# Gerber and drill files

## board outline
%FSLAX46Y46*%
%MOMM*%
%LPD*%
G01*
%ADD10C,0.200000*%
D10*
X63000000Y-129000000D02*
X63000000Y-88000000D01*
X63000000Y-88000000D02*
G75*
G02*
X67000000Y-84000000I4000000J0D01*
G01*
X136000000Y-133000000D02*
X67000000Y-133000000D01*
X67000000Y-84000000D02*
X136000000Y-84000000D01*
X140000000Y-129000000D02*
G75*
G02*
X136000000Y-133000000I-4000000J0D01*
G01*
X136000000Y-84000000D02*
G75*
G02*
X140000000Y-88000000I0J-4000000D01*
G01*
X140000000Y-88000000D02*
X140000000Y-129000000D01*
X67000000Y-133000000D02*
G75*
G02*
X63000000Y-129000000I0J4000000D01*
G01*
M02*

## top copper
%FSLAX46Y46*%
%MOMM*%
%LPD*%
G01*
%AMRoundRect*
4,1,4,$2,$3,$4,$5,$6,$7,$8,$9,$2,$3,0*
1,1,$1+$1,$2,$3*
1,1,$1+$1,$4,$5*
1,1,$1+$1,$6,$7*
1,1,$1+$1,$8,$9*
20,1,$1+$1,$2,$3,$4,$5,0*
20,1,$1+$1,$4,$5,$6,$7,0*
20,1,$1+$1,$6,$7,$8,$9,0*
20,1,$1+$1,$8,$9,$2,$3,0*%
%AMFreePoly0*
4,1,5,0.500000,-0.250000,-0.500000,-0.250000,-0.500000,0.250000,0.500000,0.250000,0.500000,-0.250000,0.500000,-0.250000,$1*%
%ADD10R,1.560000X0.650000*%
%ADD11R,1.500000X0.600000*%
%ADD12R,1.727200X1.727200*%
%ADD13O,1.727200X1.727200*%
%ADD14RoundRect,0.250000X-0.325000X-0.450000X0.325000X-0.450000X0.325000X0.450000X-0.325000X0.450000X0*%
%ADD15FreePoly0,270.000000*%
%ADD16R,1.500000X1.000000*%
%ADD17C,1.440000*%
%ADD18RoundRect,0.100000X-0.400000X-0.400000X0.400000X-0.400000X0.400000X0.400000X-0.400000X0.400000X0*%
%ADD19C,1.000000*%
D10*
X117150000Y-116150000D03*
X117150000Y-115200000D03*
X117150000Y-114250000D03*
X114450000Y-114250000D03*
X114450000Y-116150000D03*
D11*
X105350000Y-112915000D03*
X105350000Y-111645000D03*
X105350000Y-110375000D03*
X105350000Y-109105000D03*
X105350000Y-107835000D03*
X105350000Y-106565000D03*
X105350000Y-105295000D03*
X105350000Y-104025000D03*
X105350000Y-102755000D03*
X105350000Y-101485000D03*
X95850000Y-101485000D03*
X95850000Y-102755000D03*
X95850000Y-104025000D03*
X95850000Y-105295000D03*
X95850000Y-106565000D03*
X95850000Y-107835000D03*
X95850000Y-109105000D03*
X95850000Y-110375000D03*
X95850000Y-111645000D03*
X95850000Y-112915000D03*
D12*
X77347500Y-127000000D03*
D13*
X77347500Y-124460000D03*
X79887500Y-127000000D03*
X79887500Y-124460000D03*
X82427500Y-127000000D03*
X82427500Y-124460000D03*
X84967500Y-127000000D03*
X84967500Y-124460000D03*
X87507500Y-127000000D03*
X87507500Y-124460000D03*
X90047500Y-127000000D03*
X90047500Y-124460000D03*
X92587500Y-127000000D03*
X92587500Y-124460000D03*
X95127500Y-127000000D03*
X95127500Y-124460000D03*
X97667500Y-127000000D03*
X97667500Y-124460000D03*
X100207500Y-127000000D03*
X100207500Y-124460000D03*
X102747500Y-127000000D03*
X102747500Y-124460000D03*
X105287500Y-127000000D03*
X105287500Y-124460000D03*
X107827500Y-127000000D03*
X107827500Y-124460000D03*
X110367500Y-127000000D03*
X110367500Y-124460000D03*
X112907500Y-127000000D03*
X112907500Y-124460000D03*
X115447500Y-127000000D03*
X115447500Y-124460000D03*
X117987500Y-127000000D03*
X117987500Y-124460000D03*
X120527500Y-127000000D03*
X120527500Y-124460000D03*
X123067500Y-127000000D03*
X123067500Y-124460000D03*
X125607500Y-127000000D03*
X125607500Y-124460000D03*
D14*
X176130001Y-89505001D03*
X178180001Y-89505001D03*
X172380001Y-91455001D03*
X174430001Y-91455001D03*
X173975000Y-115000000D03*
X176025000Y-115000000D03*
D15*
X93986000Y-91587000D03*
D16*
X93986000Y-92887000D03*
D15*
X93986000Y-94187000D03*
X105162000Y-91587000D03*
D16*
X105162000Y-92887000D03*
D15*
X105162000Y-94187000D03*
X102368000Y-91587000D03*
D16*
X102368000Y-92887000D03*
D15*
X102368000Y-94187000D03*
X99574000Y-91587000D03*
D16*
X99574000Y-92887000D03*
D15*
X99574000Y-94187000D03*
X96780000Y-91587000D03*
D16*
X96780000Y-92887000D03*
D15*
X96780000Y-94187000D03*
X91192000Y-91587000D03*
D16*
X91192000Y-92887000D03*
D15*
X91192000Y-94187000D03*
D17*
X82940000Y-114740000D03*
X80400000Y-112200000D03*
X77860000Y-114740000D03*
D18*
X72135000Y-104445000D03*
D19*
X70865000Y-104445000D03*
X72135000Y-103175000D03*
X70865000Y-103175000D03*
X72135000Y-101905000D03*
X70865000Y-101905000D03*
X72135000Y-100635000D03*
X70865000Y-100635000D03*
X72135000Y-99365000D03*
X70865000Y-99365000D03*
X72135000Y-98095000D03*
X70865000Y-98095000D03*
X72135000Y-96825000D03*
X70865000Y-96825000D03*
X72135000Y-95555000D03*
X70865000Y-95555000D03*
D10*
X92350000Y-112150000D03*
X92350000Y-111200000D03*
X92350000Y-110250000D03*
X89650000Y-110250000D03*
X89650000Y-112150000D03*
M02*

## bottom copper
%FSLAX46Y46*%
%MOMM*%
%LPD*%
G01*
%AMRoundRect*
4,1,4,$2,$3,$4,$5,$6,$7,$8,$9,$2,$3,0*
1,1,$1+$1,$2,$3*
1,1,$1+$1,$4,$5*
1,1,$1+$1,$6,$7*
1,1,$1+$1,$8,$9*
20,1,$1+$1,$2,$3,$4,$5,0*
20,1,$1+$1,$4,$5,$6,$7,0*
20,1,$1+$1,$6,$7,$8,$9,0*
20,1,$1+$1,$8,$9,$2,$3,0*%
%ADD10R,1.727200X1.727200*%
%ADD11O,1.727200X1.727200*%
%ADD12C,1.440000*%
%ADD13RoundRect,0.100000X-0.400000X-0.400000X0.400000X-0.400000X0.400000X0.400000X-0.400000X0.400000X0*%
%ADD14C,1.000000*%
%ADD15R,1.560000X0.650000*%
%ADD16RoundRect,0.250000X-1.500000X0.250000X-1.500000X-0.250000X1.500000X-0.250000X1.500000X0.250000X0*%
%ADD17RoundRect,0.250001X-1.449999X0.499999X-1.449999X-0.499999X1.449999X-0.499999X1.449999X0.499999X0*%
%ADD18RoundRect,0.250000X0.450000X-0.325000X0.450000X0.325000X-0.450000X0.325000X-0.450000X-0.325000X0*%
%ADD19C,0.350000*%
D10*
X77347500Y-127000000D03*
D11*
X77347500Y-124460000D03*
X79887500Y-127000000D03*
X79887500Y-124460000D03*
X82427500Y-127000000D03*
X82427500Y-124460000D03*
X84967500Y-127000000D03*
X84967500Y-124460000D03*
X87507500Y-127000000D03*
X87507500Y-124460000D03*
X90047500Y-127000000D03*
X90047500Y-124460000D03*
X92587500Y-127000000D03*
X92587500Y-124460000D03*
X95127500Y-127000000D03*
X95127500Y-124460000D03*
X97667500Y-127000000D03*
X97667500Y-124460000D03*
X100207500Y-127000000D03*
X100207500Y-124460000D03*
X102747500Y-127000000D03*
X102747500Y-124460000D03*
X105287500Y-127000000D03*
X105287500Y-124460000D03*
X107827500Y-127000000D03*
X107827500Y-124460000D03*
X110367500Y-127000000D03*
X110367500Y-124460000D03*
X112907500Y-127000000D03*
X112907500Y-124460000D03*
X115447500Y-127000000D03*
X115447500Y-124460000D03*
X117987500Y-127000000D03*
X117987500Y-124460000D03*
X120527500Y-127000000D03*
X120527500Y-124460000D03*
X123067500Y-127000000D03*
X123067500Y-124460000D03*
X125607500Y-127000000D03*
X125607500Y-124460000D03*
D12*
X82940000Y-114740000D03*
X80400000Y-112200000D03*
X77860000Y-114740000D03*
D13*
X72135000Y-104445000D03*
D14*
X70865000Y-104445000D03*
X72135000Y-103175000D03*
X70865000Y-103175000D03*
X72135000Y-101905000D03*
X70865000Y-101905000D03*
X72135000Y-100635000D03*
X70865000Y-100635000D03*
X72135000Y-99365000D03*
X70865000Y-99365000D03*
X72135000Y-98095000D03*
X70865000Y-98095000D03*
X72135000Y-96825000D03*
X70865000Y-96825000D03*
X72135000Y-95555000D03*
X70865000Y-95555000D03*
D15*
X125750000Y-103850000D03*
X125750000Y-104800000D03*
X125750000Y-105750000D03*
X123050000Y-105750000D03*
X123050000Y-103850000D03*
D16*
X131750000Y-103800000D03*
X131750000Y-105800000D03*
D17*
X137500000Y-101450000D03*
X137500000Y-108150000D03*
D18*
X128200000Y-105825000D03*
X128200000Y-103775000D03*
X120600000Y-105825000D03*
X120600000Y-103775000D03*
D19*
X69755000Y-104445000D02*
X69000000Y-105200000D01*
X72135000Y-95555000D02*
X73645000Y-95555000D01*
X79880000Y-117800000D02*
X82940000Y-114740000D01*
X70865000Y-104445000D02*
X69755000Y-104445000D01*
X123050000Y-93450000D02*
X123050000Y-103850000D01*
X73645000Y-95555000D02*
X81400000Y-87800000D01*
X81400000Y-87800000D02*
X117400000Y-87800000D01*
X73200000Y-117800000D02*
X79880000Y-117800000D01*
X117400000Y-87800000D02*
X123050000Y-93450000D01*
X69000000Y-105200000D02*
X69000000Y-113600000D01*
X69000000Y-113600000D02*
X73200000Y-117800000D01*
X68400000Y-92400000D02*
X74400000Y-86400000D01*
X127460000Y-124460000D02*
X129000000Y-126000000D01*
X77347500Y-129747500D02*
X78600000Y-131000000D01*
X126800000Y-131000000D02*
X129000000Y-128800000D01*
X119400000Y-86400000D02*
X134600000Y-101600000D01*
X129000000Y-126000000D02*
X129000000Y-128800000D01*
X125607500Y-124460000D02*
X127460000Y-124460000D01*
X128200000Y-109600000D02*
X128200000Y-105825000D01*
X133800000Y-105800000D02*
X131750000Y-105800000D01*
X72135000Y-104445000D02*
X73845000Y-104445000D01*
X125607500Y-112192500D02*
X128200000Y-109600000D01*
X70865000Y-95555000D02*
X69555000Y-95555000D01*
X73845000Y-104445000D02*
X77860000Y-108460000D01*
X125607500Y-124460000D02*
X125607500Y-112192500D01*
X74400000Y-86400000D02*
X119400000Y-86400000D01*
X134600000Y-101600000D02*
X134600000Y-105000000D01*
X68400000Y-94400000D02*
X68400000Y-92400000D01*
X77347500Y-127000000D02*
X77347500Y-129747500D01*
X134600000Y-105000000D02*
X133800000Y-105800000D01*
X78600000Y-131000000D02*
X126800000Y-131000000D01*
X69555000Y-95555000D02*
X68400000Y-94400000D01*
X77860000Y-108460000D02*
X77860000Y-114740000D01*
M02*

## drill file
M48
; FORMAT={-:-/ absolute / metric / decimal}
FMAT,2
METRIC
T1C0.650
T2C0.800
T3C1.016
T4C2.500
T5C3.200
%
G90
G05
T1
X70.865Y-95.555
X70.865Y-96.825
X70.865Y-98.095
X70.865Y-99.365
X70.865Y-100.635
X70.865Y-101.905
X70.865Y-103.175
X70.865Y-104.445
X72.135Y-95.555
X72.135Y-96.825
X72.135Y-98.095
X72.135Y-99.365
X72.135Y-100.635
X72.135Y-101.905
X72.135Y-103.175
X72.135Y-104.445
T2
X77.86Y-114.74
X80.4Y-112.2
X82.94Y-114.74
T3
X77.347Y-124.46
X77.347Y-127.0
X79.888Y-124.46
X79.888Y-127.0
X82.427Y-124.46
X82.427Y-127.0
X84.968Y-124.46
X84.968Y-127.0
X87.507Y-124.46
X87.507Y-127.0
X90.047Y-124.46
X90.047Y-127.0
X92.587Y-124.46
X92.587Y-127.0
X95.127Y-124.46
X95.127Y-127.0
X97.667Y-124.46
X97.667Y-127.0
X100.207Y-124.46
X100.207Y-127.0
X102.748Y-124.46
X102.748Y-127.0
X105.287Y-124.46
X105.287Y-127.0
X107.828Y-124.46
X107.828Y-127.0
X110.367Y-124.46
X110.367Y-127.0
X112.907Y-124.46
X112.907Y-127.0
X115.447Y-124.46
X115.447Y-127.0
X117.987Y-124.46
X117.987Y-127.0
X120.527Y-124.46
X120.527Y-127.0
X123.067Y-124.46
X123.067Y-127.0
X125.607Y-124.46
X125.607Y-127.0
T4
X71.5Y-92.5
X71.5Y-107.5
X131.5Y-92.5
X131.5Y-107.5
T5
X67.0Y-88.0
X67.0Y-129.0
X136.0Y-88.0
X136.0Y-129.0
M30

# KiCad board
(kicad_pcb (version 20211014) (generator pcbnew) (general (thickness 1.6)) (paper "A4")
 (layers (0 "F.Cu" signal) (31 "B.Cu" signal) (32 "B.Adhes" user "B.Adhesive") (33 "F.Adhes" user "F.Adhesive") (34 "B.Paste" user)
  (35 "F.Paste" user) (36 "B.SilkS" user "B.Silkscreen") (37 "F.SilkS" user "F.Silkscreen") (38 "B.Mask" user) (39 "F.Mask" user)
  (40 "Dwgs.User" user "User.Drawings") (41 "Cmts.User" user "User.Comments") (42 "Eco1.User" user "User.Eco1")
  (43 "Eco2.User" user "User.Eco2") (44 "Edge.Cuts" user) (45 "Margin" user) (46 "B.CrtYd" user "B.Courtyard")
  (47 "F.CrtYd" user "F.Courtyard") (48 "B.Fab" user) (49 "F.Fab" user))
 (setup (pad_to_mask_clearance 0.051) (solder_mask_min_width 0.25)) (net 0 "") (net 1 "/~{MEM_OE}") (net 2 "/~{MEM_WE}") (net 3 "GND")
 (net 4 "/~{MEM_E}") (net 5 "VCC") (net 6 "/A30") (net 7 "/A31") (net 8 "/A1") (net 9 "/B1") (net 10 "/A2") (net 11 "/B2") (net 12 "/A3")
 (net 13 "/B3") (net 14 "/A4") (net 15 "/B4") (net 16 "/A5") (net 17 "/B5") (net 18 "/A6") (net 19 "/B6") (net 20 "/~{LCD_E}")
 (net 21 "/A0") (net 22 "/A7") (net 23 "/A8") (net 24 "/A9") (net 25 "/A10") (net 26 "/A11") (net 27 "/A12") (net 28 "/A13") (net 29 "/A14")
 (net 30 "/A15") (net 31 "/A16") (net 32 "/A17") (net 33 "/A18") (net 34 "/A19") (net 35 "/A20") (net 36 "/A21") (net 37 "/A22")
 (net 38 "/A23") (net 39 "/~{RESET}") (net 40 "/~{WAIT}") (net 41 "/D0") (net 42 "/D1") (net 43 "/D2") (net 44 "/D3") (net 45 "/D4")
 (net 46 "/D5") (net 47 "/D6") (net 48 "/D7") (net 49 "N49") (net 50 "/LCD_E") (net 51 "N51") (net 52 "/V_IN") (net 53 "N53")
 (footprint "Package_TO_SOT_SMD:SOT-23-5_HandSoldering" (layer "F.Cu") (at 115.8 115.2 180)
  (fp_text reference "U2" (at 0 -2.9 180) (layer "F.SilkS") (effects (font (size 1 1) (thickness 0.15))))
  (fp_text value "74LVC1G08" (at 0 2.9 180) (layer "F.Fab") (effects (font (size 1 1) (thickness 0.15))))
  (pad "1" smd rect locked (at -1.35 -0.95 180) (size 1.56 0.65) (layers "F.Cu" "F.Paste" "F.Mask") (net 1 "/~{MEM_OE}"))
  (pad "2" smd rect locked (at -1.35 0 180) (size 1.56 0.65) (layers "F.Cu" "F.Paste" "F.Mask") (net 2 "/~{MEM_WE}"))
  (pad "3" smd rect locked (at -1.35 0.95 180) (size 1.56 0.65) (layers "F.Cu" "F.Paste" "F.Mask") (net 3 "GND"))
  (pad "4" smd rect locked (at 1.35 0.95 180) (size 1.56 0.65) (layers "F.Cu" "F.Paste" "F.Mask") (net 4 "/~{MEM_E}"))
  (pad "5" smd rect locked (at 1.35 -0.95 180) (size 1.56 0.65) (layers "F.Cu" "F.Paste" "F.Mask") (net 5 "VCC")))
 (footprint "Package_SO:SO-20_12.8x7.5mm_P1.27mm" (layer "F.Cu") (at 100.6 107.2 180)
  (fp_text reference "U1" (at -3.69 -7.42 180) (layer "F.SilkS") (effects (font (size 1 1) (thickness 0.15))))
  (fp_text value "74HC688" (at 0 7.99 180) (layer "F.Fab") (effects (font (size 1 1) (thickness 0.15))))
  (pad "1" smd rect locked (at -4.75 -5.715 180) (size 1.5 0.6) (layers "F.Cu" "F.Paste" "F.Mask") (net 4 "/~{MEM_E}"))
  (pad "2" smd rect locked (at -4.75 -4.445 180) (size 1.5 0.6) (layers "F.Cu" "F.Paste" "F.Mask") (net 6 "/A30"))
  (pad "3" smd rect locked (at -4.75 -3.175 180) (size 1.5 0.6) (layers "F.Cu" "F.Paste" "F.Mask") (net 5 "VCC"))
  (pad "4" smd rect locked (at -4.75 -1.905 180) (size 1.5 0.6) (layers "F.Cu" "F.Paste" "F.Mask") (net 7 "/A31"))
  (pad "5" smd rect locked (at -4.75 -0.635 180) (size 1.5 0.6) (layers "F.Cu" "F.Paste" "F.Mask") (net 3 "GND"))
  (pad "6" smd rect locked (at -4.75 0.635 180) (size 1.5 0.6) (layers "F.Cu" "F.Paste" "F.Mask") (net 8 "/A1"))
  (pad "7" smd rect locked (at -4.75 1.905 180) (size 1.5 0.6) (layers "F.Cu" "F.Paste" "F.Mask") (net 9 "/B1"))
  (pad "8" smd rect locked (at -4.75 3.175 180) (size 1.5 0.6) (layers "F.Cu" "F.Paste" "F.Mask") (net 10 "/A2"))
  (pad "9" smd rect locked (at -4.75 4.445 180) (size 1.5 0.6) (layers "F.Cu" "F.Paste" "F.Mask") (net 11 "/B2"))
  (pad "10" smd rect locked (at -4.75 5.715 180) (size 1.5 0.6) (layers "F.Cu" "F.Paste" "F.Mask") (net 3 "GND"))
  (pad "11" smd rect locked (at 4.75 5.715 180) (size 1.5 0.6) (layers "F.Cu" "F.Paste" "F.Mask") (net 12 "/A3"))
  (pad "12" smd rect locked (at 4.75 4.445 180) (size 1.5 0.6) (layers "F.Cu" "F.Paste" "F.Mask") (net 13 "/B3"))
  (pad "13" smd rect locked (at 4.75 3.175 180) (size 1.5 0.6) (layers "F.Cu" "F.Paste" "F.Mask") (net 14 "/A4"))
  (pad "14" smd rect locked (at 4.75 1.905 180) (size 1.5 0.6) (layers "F.Cu" "F.Paste" "F.Mask") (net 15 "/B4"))
  (pad "15" smd rect locked (at 4.75 0.635 180) (size 1.5 0.6) (layers "F.Cu" "F.Paste" "F.Mask") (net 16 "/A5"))
  (pad "16" smd rect locked (at 4.75 -0.635 180) (size 1.5 0.6) (layers "F.Cu" "F.Paste" "F.Mask") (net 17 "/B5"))
  (pad "17" smd rect locked (at 4.75 -1.905 180) (size 1.5 0.6) (layers "F.Cu" "F.Paste" "F.Mask") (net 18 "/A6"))
  (pad "18" smd rect locked (at 4.75 -3.175 180) (size 1.5 0.6) (layers "F.Cu" "F.Paste" "F.Mask") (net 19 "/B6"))
  (pad "19" smd rect locked (at 4.75 -4.445 180) (size 1.5 0.6) (layers "F.Cu" "F.Paste" "F.Mask") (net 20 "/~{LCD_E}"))
  (pad "20" smd rect locked (at 4.75 -5.715 180) (size 1.5 0.6) (layers "F.Cu" "F.Paste" "F.Mask") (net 5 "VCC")))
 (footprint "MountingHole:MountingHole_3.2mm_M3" (layer "F.Cu") (at 67 129)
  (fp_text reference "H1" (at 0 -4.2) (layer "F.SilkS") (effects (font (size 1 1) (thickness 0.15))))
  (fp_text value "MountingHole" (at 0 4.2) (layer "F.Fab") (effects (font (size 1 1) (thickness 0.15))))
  (pad "" np_thru_hole circle locked (at 0 0) (size 3.2 3.2) (drill 3.2) (layers *.Cu *.Mask)))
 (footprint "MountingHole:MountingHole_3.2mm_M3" (layer "F.Cu") (at 67 88)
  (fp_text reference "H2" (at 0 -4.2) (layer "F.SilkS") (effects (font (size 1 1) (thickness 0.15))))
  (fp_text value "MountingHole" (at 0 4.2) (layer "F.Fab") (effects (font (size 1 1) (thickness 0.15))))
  (pad "" np_thru_hole circle locked (at 0 0) (size 3.2 3.2) (drill 3.2) (layers *.Cu *.Mask)))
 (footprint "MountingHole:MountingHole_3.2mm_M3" (layer "F.Cu") (at 136 88)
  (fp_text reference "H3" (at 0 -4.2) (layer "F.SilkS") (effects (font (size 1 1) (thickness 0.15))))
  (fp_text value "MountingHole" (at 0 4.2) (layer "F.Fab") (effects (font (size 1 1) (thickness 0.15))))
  (pad "" np_thru_hole circle locked (at 0 0) (size 3.2 3.2) (drill 3.2) (layers *.Cu *.Mask)))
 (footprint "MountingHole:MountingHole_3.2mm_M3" (layer "F.Cu") (at 136 129)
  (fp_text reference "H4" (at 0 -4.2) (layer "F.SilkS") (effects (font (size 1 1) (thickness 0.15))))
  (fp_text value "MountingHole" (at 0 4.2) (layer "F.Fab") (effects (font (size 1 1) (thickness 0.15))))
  (pad "" np_thru_hole circle locked (at 0 0) (size 3.2 3.2) (drill 3.2) (layers *.Cu *.Mask)))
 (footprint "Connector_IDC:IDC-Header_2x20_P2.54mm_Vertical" (layer "F.Cu") (at 77.3475 127 90)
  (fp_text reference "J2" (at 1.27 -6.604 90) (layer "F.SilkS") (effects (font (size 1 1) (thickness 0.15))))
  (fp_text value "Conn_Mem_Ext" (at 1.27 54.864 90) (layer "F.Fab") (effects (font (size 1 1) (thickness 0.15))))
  (pad "1" thru_hole rect locked (at 0 0 90) (size 1.7272 1.7272) (drill 1.016) (layers *.Cu *.Mask) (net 3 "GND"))
  (pad "2" thru_hole oval locked (at 2.54 0 90) (size 1.7272 1.7272) (drill 1.016) (layers *.Cu *.Mask) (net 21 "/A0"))
  (pad "3" thru_hole oval locked (at 0 2.54 90) (size 1.7272 1.7272) (drill 1.016) (layers *.Cu *.Mask) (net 8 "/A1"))
  (pad "4" thru_hole oval locked (at 2.54 2.54 90) (size 1.7272 1.7272) (drill 1.016) (layers *.Cu *.Mask) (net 10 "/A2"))
  (pad "5" thru_hole oval locked (at 0 5.08 90) (size 1.7272 1.7272) (drill 1.016) (layers *.Cu *.Mask) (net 12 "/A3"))
  (pad "6" thru_hole oval locked (at 2.54 5.08 90) (size 1.7272 1.7272) (drill 1.016) (layers *.Cu *.Mask) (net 14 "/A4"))
  (pad "7" thru_hole oval locked (at 0 7.62 90) (size 1.7272 1.7272) (drill 1.016) (layers *.Cu *.Mask) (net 16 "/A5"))
  (pad "8" thru_hole oval locked (at 2.54 7.62 90) (size 1.7272 1.7272) (drill 1.016) (layers *.Cu *.Mask) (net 18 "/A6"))
  (pad "9" thru_hole oval locked (at 0 10.16 90) (size 1.7272 1.7272) (drill 1.016) (layers *.Cu *.Mask) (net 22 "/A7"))
  (pad "10" thru_hole oval locked (at 2.54 10.16 90) (size 1.7272 1.7272) (drill 1.016) (layers *.Cu *.Mask) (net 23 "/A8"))
  (pad "11" thru_hole oval locked (at 0 12.7 90) (size 1.7272 1.7272) (drill 1.016) (layers *.Cu *.Mask) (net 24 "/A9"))
  (pad "12" thru_hole oval locked (at 2.54 12.7 90) (size 1.7272 1.7272) (drill 1.016) (layers *.Cu *.Mask) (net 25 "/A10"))
  (pad "13" thru_hole oval locked (at 0 15.24 90) (size 1.7272 1.7272) (drill 1.016) (layers *.Cu *.Mask) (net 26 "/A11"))
  (pad "14" thru_hole oval locked (at 2.54 15.24 90) (size 1.7272 1.7272) (drill 1.016) (layers *.Cu *.Mask) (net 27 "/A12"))
  (pad "15" thru_hole oval locked (at 0 17.78 90) (size 1.7272 1.7272) (drill 1.016) (layers *.Cu *.Mask) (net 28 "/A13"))
  (pad "16" thru_hole oval locked (at 2.54 17.78 90) (size 1.7272 1.7272) (drill 1.016) (layers *.Cu *.Mask) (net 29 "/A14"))
  (pad "17" thru_hole oval locked (at 0 20.32 90) (size 1.7272 1.7272) (drill 1.016) (layers *.Cu *.Mask) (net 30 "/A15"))
  (pad "18" thru_hole oval locked (at 2.54 20.32 90) (size 1.7272 1.7272) (drill 1.016) (layers *.Cu *.Mask) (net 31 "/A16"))
  (pad "19" thru_hole oval locked (at 0 22.86 90) (size 1.7272 1.7272) (drill 1.016) (layers *.Cu *.Mask) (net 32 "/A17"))
  (pad "20" thru_hole oval locked (at 2.54 22.86 90) (size 1.7272 1.7272) (drill 1.016) (layers *.Cu *.Mask) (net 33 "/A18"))
  (pad "21" thru_hole oval locked (at 0 25.4 90) (size 1.7272 1.7272) (drill 1.016) (layers *.Cu *.Mask) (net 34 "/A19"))
  (pad "22" thru_hole oval locked (at 2.54 25.4 90) (size 1.7272 1.7272) (drill 1.016) (layers *.Cu *.Mask) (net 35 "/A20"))
  (pad "23" thru_hole oval locked (at 0 27.94 90) (size 1.7272 1.7272) (drill 1.016) (layers *.Cu *.Mask) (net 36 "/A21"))
  (pad "24" thru_hole oval locked (at 2.54 27.94 90) (size 1.7272 1.7272) (drill 1.016) (layers *.Cu *.Mask) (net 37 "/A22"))
  (pad "25" thru_hole oval locked (at 0 30.48 90) (size 1.7272 1.7272) (drill 1.016) (layers *.Cu *.Mask) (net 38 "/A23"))
  (pad "26" thru_hole oval locked (at 2.54 30.48 90) (size 1.7272 1.7272) (drill 1.016) (layers *.Cu *.Mask) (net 6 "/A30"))
  (pad "27" thru_hole oval locked (at 0 33.02 90) (size 1.7272 1.7272) (drill 1.016) (layers *.Cu *.Mask) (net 7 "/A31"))
  (pad "28" thru_hole oval locked (at 2.54 33.02 90) (size 1.7272 1.7272) (drill 1.016) (layers *.Cu *.Mask) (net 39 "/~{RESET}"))
  (pad "29" thru_hole oval locked (at 0 35.56 90) (size 1.7272 1.7272) (drill 1.016) (layers *.Cu *.Mask) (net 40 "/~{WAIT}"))
  (pad "30" thru_hole oval locked (at 2.54 35.56 90) (size 1.7272 1.7272) (drill 1.016) (layers *.Cu *.Mask) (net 1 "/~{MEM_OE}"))
  (pad "31" thru_hole oval locked (at 0 38.1 90) (size 1.7272 1.7272) (drill 1.016) (layers *.Cu *.Mask) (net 2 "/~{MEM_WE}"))
  (pad "32" thru_hole oval locked (at 2.54 38.1 90) (size 1.7272 1.7272) (drill 1.016) (layers *.Cu *.Mask) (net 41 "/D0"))
  (pad "33" thru_hole oval locked (at 0 40.64 90) (size 1.7272 1.7272) (drill 1.016) (layers *.Cu *.Mask) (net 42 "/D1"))
  (pad "34" thru_hole oval locked (at 2.54 40.64 90) (size 1.7272 1.7272) (drill 1.016) (layers *.Cu *.Mask) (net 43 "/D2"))
  (pad "35" thru_hole oval locked (at 0 43.18 90) (size 1.7272 1.7272) (drill 1.016) (layers *.Cu *.Mask) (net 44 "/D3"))
  (pad "36" thru_hole oval locked (at 2.54 43.18 90) (size 1.7272 1.7272) (drill 1.016) (layers *.Cu *.Mask) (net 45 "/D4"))
  (pad "37" thru_hole oval locked (at 0 45.72 90) (size 1.7272 1.7272) (drill 1.016) (layers *.Cu *.Mask) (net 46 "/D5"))
  (pad "38" thru_hole oval locked (at 2.54 45.72 90) (size 1.7272 1.7272) (drill 1.016) (layers *.Cu *.Mask) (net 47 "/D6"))
  (pad "39" thru_hole oval locked (at 0 48.26 90) (size 1.7272 1.7272) (drill 1.016) (layers *.Cu *.Mask) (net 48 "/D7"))
  (pad "40" thru_hole oval locked (at 2.54 48.26 90) (size 1.7272 1.7272) (drill 1.016) (layers *.Cu *.Mask) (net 3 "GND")))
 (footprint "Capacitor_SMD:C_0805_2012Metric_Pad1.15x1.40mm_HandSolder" (layer "F.Cu") (at 177.155001 89.505001)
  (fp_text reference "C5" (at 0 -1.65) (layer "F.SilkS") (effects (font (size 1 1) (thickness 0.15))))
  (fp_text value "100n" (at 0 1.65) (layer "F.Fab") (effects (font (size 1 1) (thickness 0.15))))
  (pad "1" smd roundrect locked (at -1.025 0) (size 1.15 1.4) (layers "F.Cu" "F.Paste" "F.Mask") (roundrect_rratio 0.217391) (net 3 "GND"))
  (pad "2" smd roundrect locked (at 1.025 0) (size 1.15 1.4) (layers "F.Cu" "F.Paste" "F.Mask") (roundrect_rratio 0.217391) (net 5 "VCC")))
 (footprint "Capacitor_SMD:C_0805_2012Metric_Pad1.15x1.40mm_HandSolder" (layer "F.Cu") (at 173.405001 91.455001)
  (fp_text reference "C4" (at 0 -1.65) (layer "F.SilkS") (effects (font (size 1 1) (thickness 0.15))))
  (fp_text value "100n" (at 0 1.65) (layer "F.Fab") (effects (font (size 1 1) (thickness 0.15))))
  (pad "1" smd roundrect locked (at -1.025 0) (size 1.15 1.4) (layers "F.Cu" "F.Paste" "F.Mask") (roundrect_rratio 0.217391) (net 3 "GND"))
  (pad "2" smd roundrect locked (at 1.025 0) (size 1.15 1.4) (layers "F.Cu" "F.Paste" "F.Mask") (roundrect_rratio 0.217391) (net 5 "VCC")))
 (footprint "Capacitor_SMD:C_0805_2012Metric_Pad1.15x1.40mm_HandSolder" (layer "F.Cu") (at 175 115)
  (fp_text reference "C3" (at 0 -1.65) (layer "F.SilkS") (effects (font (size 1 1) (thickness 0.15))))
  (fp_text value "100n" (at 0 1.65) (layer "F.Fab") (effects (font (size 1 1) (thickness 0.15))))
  (pad "1" smd roundrect locked (at -1.025 0) (size 1.15 1.4) (layers "F.Cu" "F.Paste" "F.Mask") (roundrect_rratio 0.217391) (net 3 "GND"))
  (pad "2" smd roundrect locked (at 1.025 0) (size 1.15 1.4) (layers "F.Cu" "F.Paste" "F.Mask") (roundrect_rratio 0.217391) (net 5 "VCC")))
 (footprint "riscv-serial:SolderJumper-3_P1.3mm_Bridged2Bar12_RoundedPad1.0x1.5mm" (layer "F.Cu") (at 93.986 92.887 -90)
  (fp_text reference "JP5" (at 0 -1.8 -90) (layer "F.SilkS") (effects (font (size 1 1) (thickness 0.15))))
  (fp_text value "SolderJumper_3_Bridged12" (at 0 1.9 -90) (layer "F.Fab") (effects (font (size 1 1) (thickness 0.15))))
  (pad "1" smd custom locked (at -1.3 0 270) (size 1 0.5) (layers "F.Cu" "F.Mask") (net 3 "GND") (zone_connect 0)
   (options (clearance outline) (anchor rect)) (primitives))
  (pad "2" smd rect locked (at 0 0 270) (size 1 1.5) (layers "F.Cu" "F.Mask") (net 17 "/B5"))
  (pad "3" smd custom locked (at 1.3 0 270) (size 1 0.5) (layers "F.Cu" "F.Mask") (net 5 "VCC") (zone_connect 0)
   (options (clearance outline) (anchor rect)) (primitives)))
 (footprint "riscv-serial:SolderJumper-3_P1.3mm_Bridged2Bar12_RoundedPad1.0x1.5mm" (layer "F.Cu") (at 105.162 92.887 -90)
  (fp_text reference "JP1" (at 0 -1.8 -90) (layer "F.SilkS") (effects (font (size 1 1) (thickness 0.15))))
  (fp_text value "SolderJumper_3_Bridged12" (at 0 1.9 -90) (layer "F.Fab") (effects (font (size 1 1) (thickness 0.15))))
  (pad "1" smd custom locked (at -1.3 0 270) (size 1 0.5) (layers "F.Cu" "F.Mask") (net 3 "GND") (zone_connect 0)
   (options (clearance outline) (anchor rect)) (primitives))
  (pad "2" smd rect locked (at 0 0 270) (size 1 1.5) (layers "F.Cu" "F.Mask") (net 9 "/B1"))
  (pad "3" smd custom locked (at 1.3 0 270) (size 1 0.5) (layers "F.Cu" "F.Mask") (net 5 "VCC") (zone_connect 0)
   (options (clearance outline) (anchor rect)) (primitives)))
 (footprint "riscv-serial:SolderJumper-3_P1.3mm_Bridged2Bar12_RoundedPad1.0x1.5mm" (layer "F.Cu") (at 102.368 92.887 -90)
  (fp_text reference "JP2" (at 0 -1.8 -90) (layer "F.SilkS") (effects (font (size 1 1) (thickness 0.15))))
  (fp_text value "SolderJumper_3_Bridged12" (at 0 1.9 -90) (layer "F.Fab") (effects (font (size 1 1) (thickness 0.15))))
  (pad "1" smd custom locked (at -1.3 0 270) (size 1 0.5) (layers "F.Cu" "F.Mask") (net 3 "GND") (zone_connect 0)
   (options (clearance outline) (anchor rect)) (primitives))
  (pad "2" smd rect locked (at 0 0 270) (size 1 1.5) (layers "F.Cu" "F.Mask") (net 11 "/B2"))
  (pad "3" smd custom locked (at 1.3 0 270) (size 1 0.5) (layers "F.Cu" "F.Mask") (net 5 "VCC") (zone_connect 0)
   (options (clearance outline) (anchor rect)) (primitives)))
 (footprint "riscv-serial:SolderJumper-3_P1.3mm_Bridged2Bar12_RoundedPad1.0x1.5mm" (layer "F.Cu") (at 99.574 92.887 -90)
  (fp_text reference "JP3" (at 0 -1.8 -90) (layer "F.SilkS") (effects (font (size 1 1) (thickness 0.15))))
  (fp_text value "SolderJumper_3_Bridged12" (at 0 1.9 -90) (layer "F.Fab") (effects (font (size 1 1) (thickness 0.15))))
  (pad "1" smd custom locked (at -1.3 0 270) (size 1 0.5) (layers "F.Cu" "F.Mask") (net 3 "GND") (zone_connect 0)
   (options (clearance outline) (anchor rect)) (primitives))
  (pad "2" smd rect locked (at 0 0 270) (size 1 1.5) (layers "F.Cu" "F.Mask") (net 13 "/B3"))
  (pad "3" smd custom locked (at 1.3 0 270) (size 1 0.5) (layers "F.Cu" "F.Mask") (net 5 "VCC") (zone_connect 0)
   (options (clearance outline) (anchor rect)) (primitives)))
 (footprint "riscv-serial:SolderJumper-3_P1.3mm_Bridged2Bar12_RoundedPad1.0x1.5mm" (layer "F.Cu") (at 96.78 92.887 -90)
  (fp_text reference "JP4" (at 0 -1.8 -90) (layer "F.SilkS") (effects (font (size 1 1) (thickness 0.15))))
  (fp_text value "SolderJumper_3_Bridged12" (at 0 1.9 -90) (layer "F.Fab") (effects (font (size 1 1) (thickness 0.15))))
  (pad "1" smd custom locked (at -1.3 0 270) (size 1 0.5) (layers "F.Cu" "F.Mask") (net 3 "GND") (zone_connect 0)
   (options (clearance outline) (anchor rect)) (primitives))
  (pad "2" smd rect locked (at 0 0 270) (size 1 1.5) (layers "F.Cu" "F.Mask") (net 15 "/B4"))
  (pad "3" smd custom locked (at 1.3 0 270) (size 1 0.5) (layers "F.Cu" "F.Mask") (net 5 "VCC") (zone_connect 0)
   (options (clearance outline) (anchor rect)) (primitives)))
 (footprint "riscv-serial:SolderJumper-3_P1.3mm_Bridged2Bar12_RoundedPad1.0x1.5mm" (layer "F.Cu") (at 91.192 92.887 -90)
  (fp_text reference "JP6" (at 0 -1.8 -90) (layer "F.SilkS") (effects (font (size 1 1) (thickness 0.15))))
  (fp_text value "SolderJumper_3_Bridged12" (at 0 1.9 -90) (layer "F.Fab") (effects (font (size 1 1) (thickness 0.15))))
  (pad "1" smd custom locked (at -1.3 0 270) (size 1 0.5) (layers "F.Cu" "F.Mask") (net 3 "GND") (zone_connect 0)
   (options (clearance outline) (anchor rect)) (primitives))
  (pad "2" smd rect locked (at 0 0 270) (size 1 1.5) (layers "F.Cu" "F.Mask") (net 19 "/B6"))
  (pad "3" smd custom locked (at 1.3 0 270) (size 1 0.5) (layers "F.Cu" "F.Mask") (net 5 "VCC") (zone_connect 0)
   (options (clearance outline) (anchor rect)) (primitives)))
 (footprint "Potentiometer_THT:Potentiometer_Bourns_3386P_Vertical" (layer "F.Cu") (at 82.94 114.74 90)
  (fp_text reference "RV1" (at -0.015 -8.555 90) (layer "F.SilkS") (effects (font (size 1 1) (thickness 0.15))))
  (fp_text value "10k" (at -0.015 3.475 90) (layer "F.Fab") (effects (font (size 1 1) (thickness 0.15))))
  (pad "1" thru_hole circle locked (at 0 0 90) (size 1.44 1.44) (drill 0.8) (layers *.Cu *.Mask) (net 5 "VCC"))
  (pad "2" thru_hole circle locked (at 2.54 -2.54 90) (size 1.44 1.44) (drill 0.8) (layers *.Cu *.Mask) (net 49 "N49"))
  (pad "3" thru_hole circle locked (at 0 -5.08 90) (size 1.44 1.44) (drill 0.8) (layers *.Cu *.Mask) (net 3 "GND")))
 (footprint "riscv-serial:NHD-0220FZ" (layer "F.Cu") (at 101.5 100)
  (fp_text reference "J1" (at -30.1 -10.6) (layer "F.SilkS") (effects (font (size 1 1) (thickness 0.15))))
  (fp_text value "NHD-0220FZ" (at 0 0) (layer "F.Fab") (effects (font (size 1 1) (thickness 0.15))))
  (pad "" np_thru_hole circle locked (at 30 7.5) (size 2.5 2.5) (drill 2.5) (layers *.Cu *.Mask))
  (pad "" np_thru_hole circle locked (at 30 -7.5) (size 2.5 2.5) (drill 2.5) (layers *.Cu *.Mask))
  (pad "" np_thru_hole circle locked (at -30 -7.5) (size 2.5 2.5) (drill 2.5) (layers *.Cu *.Mask))
  (pad "" np_thru_hole circle locked (at -30 7.5) (size 2.5 2.5) (drill 2.5) (layers *.Cu *.Mask))
  (pad "1" thru_hole roundrect locked (at -29.365 4.445) (size 1 1) (drill 0.65) (layers *.Cu *.Mask) (roundrect_rratio 0.1) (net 3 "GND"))
  (pad "2" thru_hole circle locked (at -30.635 4.445) (size 1 1) (drill 0.65) (layers *.Cu *.Mask) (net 5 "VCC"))
  (pad "3" thru_hole circle locked (at -29.365 3.175) (size 1 1) (drill 0.65) (layers *.Cu *.Mask) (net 49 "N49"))
  (pad "4" thru_hole circle locked (at -30.635 3.175) (size 1 1) (drill 0.65) (layers *.Cu *.Mask) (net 21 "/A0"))
  (pad "5" thru_hole circle locked (at -29.365 1.905) (size 1 1) (drill 0.65) (layers *.Cu *.Mask) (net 2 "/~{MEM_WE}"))
  (pad "6" thru_hole circle locked (at -30.635 1.905) (size 1 1) (drill 0.65) (layers *.Cu *.Mask) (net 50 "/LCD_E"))
  (pad "7" thru_hole circle locked (at -29.365 0.635) (size 1 1) (drill 0.65) (layers *.Cu *.Mask) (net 48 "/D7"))
  (pad "8" thru_hole circle locked (at -30.635 0.635) (size 1 1) (drill 0.65) (layers *.Cu *.Mask) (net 47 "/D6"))
  (pad "9" thru_hole circle locked (at -29.365 -0.635) (size 1 1) (drill 0.65) (layers *.Cu *.Mask) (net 46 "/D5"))
  (pad "10" thru_hole circle locked (at -30.635 -0.635) (size 1 1) (drill 0.65) (layers *.Cu *.Mask) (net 45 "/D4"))
  (pad "11" thru_hole circle locked (at -29.365 -1.905) (size 1 1) (drill 0.65) (layers *.Cu *.Mask) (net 44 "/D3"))
  (pad "12" thru_hole circle locked (at -30.635 -1.905) (size 1 1) (drill 0.65) (layers *.Cu *.Mask) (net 43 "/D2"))
  (pad "13" thru_hole circle locked (at -29.365 -3.175) (size 1 1) (drill 0.65) (layers *.Cu *.Mask) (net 42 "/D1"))
  (pad "14" thru_hole circle locked (at -30.635 -3.175) (size 1 1) (drill 0.65) (layers *.Cu *.Mask) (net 41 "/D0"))
  (pad "15" thru_hole circle locked (at -29.365 -4.445) (size 1 1) (drill 0.65) (layers *.Cu *.Mask) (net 5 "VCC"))
  (pad "16" thru_hole circle locked (at -30.635 -4.445) (size 1 1) (drill 0.65) (layers *.Cu *.Mask) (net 3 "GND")))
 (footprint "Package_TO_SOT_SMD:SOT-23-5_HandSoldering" (layer "F.Cu") (at 91 111.2 180)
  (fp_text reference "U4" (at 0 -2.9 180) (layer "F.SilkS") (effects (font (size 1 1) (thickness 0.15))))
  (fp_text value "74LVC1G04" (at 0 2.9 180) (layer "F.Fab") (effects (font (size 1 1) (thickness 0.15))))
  (pad "1" smd rect locked (at -1.35 -0.95 180) (size 1.56 0.65) (layers "F.Cu" "F.Paste" "F.Mask") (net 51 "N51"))
  (pad "2" smd rect locked (at -1.35 0 180) (size 1.56 0.65) (layers "F.Cu" "F.Paste" "F.Mask") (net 20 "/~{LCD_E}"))
  (pad "3" smd rect locked (at -1.35 0.95 180) (size 1.56 0.65) (layers "F.Cu" "F.Paste" "F.Mask") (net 3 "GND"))
  (pad "4" smd rect locked (at 1.35 0.95 180) (size 1.56 0.65) (layers "F.Cu" "F.Paste" "F.Mask") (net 50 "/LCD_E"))
  (pad "5" smd rect locked (at 1.35 -0.95 180) (size 1.56 0.65) (layers "F.Cu" "F.Paste" "F.Mask") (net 5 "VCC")))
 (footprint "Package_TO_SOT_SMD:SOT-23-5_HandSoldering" (layer "B.Cu") (at 124.4 104.8 180)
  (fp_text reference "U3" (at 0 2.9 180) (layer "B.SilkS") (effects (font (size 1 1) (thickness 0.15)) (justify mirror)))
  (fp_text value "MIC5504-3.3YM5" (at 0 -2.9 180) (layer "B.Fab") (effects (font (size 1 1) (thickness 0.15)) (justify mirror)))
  (pad "1" smd rect locked (at -1.35 0.95 180) (size 1.56 0.65) (layers "B.Cu" "B.Paste" "B.Mask") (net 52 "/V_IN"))
  (pad "2" smd rect locked (at -1.35 0 180) (size 1.56 0.65) (layers "B.Cu" "B.Paste" "B.Mask") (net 3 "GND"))
  (pad "3" smd rect locked (at -1.35 -0.95 180) (size 1.56 0.65) (layers "B.Cu" "B.Paste" "B.Mask") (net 52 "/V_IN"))
  (pad "4" smd rect locked (at 1.35 -0.95 180) (size 1.56 0.65) (layers "B.Cu" "B.Paste" "B.Mask") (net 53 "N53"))
  (pad "5" smd rect locked (at 1.35 0.95 180) (size 1.56 0.65) (layers "B.Cu" "B.Paste" "B.Mask") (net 5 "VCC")))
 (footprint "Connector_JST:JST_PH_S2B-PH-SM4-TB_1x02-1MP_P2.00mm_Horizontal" (layer "B.Cu") (at 134.6 104.8 -90)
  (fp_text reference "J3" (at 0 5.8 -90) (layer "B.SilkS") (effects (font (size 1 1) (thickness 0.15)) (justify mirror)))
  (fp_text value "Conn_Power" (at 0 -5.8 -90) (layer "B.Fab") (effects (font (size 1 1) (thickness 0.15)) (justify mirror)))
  (pad "1" smd roundrect locked (at -1 2.85 270) (size 1 3.5) (layers "B.Cu" "B.Paste" "B.Mask") (roundrect_rratio 0.25) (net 52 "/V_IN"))
  (pad "2" smd roundrect locked (at 1 2.85 270) (size 1 3.5) (layers "B.Cu" "B.Paste" "B.Mask") (roundrect_rratio 0.25) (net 3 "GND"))
  (pad "MP" smd roundrect locked (at -3.35 -2.9 270) (size 1.5 3.4) (layers "B.Cu" "B.Paste" "B.Mask") (roundrect_rratio 0.166667)
   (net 3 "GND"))
  (pad "MP" smd roundrect locked (at 3.35 -2.9 270) (size 1.5 3.4) (layers "B.Cu" "B.Paste" "B.Mask") (roundrect_rratio 0.166667)
   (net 3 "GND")))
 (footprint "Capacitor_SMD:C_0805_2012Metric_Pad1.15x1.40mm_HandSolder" (layer "B.Cu") (at 128.2 104.8 90)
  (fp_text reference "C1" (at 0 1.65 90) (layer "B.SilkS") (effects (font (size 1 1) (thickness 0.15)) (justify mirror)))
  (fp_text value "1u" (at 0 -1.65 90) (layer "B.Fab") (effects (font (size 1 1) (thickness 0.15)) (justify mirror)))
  (pad "1" smd roundrect locked (at -1.025 0 90) (size 1.15 1.4) (layers "B.Cu" "B.Paste" "B.Mask") (roundrect_rratio 0.217391)
   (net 3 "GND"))
  (pad "2" smd roundrect locked (at 1.025 0 90) (size 1.15 1.4) (layers "B.Cu" "B.Paste" "B.Mask") (roundrect_rratio 0.217391)
   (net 52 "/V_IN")))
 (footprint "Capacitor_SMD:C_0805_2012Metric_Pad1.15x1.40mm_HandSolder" (layer "B.Cu") (at 120.6 104.8 90)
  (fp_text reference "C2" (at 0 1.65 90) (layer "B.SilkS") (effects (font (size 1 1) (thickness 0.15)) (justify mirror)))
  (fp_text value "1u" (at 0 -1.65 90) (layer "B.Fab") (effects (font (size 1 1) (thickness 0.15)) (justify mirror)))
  (pad "1" smd roundrect locked (at -1.025 0 90) (size 1.15 1.4) (layers "B.Cu" "B.Paste" "B.Mask") (roundrect_rratio 0.217391)
   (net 3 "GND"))
  (pad "2" smd roundrect locked (at 1.025 0 90) (size 1.15 1.4) (layers "B.Cu" "B.Paste" "B.Mask") (roundrect_rratio 0.217391) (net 5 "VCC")))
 (gr_line (start 63 129) (end 63 88) (layer "Edge.Cuts") (width 0.2))
 (gr_arc (start 63 88) (mid 64.171573 85.171573) (end 67 84) (layer "Edge.Cuts") (width 0.2))
 (gr_line (start 136 133) (end 67 133) (layer "Edge.Cuts") (width 0.2))
 (gr_line (start 67 84) (end 136 84) (layer "Edge.Cuts") (width 0.2))
 (gr_arc (start 140 129) (mid 138.828427 131.828427) (end 136 133) (layer "Edge.Cuts") (width 0.2))
 (gr_arc (start 136 84) (mid 138.828427 85.171573) (end 140 88) (layer "Edge.Cuts") (width 0.2))
 (gr_line (start 140 88) (end 140 129) (layer "Edge.Cuts") (width 0.2))
 (gr_arc (start 67 133) (mid 64.171573 131.828427) (end 63 129) (layer "Edge.Cuts") (width 0.2))
 (segment (start 69.755 104.445) (end 69 105.2) (width 0.35) (layer "B.Cu") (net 5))
 (segment (start 72.135 95.555) (end 73.645 95.555) (width 0.35) (layer "B.Cu") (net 5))
 (segment (start 79.88 117.8) (end 82.94 114.74) (width 0.35) (layer "B.Cu") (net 5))
 (segment (start 70.865 104.445) (end 69.755 104.445) (width 0.35) (layer "B.Cu") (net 5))
 (segment (start 123.05 93.45) (end 123.05 103.85) (width 0.35) (layer "B.Cu") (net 5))
 (segment (start 73.645 95.555) (end 81.4 87.8) (width 0.35) (layer "B.Cu") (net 5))
 (segment (start 81.4 87.8) (end 117.4 87.8) (width 0.35) (layer "B.Cu") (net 5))
 (segment (start 73.2 117.8) (end 79.88 117.8) (width 0.35) (layer "B.Cu") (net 5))
 (segment (start 117.4 87.8) (end 123.05 93.45) (width 0.35) (layer "B.Cu") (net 5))
 (segment (start 69 105.2) (end 69 113.6) (width 0.35) (layer "B.Cu") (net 5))
 (segment (start 69 113.6) (end 73.2 117.8) (width 0.35) (layer "B.Cu") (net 5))
 (segment (start 68.4 92.4) (end 74.4 86.4) (width 0.35) (layer "B.Cu") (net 3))
 (segment (start 127.46 124.46) (end 129 126) (width 0.35) (layer "B.Cu") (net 3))
 (segment (start 77.3475 129.7475) (end 78.6 131) (width 0.35) (layer "B.Cu") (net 3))
 (segment (start 126.8 131) (end 129 128.8) (width 0.35) (layer "B.Cu") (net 3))
 (segment (start 119.4 86.4) (end 134.6 101.6) (width 0.35) (layer "B.Cu") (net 3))
 (segment (start 129 126) (end 129 128.8) (width 0.35) (layer "B.Cu") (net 3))
 (segment (start 125.6075 124.46) (end 127.46 124.46) (width 0.35) (layer "B.Cu") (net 3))
 (segment (start 128.2 109.6) (end 128.2 105.825) (width 0.35) (layer "B.Cu") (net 3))
 (segment (start 133.8 105.8) (end 131.75 105.8) (width 0.35) (layer "B.Cu") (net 3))
 (segment (start 72.135 104.445) (end 73.845 104.445) (width 0.35) (layer "B.Cu") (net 3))
 (segment (start 125.6075 112.1925) (end 128.2 109.6) (width 0.35) (layer "B.Cu") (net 3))
 (segment (start 70.865 95.555) (end 69.555 95.555) (width 0.35) (layer "B.Cu") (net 3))
 (segment (start 73.845 104.445) (end 77.86 108.46) (width 0.35) (layer "B.Cu") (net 3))
 (segment (start 125.6075 124.46) (end 125.6075 112.1925) (width 0.35) (layer "B.Cu") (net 3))
 (segment (start 74.4 86.4) (end 119.4 86.4) (width 0.35) (layer "B.Cu") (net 3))
 (segment (start 134.6 101.6) (end 134.6 105) (width 0.35) (layer "B.Cu") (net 3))
 (segment (start 68.4 94.4) (end 68.4 92.4) (width 0.35) (layer "B.Cu") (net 3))
 (segment (start 77.3475 127) (end 77.3475 129.7475) (width 0.35) (layer "B.Cu") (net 3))
 (segment (start 134.6 105) (end 133.8 105.8) (width 0.35) (layer "B.Cu") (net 3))
 (segment (start 78.6 131) (end 126.8 131) (width 0.35) (layer "B.Cu") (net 3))
 (segment (start 69.555 95.555) (end 68.4 94.4) (width 0.35) (layer "B.Cu") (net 3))
 (segment (start 77.86 108.46) (end 77.86 114.74) (width 0.35) (layer "B.Cu") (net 3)))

